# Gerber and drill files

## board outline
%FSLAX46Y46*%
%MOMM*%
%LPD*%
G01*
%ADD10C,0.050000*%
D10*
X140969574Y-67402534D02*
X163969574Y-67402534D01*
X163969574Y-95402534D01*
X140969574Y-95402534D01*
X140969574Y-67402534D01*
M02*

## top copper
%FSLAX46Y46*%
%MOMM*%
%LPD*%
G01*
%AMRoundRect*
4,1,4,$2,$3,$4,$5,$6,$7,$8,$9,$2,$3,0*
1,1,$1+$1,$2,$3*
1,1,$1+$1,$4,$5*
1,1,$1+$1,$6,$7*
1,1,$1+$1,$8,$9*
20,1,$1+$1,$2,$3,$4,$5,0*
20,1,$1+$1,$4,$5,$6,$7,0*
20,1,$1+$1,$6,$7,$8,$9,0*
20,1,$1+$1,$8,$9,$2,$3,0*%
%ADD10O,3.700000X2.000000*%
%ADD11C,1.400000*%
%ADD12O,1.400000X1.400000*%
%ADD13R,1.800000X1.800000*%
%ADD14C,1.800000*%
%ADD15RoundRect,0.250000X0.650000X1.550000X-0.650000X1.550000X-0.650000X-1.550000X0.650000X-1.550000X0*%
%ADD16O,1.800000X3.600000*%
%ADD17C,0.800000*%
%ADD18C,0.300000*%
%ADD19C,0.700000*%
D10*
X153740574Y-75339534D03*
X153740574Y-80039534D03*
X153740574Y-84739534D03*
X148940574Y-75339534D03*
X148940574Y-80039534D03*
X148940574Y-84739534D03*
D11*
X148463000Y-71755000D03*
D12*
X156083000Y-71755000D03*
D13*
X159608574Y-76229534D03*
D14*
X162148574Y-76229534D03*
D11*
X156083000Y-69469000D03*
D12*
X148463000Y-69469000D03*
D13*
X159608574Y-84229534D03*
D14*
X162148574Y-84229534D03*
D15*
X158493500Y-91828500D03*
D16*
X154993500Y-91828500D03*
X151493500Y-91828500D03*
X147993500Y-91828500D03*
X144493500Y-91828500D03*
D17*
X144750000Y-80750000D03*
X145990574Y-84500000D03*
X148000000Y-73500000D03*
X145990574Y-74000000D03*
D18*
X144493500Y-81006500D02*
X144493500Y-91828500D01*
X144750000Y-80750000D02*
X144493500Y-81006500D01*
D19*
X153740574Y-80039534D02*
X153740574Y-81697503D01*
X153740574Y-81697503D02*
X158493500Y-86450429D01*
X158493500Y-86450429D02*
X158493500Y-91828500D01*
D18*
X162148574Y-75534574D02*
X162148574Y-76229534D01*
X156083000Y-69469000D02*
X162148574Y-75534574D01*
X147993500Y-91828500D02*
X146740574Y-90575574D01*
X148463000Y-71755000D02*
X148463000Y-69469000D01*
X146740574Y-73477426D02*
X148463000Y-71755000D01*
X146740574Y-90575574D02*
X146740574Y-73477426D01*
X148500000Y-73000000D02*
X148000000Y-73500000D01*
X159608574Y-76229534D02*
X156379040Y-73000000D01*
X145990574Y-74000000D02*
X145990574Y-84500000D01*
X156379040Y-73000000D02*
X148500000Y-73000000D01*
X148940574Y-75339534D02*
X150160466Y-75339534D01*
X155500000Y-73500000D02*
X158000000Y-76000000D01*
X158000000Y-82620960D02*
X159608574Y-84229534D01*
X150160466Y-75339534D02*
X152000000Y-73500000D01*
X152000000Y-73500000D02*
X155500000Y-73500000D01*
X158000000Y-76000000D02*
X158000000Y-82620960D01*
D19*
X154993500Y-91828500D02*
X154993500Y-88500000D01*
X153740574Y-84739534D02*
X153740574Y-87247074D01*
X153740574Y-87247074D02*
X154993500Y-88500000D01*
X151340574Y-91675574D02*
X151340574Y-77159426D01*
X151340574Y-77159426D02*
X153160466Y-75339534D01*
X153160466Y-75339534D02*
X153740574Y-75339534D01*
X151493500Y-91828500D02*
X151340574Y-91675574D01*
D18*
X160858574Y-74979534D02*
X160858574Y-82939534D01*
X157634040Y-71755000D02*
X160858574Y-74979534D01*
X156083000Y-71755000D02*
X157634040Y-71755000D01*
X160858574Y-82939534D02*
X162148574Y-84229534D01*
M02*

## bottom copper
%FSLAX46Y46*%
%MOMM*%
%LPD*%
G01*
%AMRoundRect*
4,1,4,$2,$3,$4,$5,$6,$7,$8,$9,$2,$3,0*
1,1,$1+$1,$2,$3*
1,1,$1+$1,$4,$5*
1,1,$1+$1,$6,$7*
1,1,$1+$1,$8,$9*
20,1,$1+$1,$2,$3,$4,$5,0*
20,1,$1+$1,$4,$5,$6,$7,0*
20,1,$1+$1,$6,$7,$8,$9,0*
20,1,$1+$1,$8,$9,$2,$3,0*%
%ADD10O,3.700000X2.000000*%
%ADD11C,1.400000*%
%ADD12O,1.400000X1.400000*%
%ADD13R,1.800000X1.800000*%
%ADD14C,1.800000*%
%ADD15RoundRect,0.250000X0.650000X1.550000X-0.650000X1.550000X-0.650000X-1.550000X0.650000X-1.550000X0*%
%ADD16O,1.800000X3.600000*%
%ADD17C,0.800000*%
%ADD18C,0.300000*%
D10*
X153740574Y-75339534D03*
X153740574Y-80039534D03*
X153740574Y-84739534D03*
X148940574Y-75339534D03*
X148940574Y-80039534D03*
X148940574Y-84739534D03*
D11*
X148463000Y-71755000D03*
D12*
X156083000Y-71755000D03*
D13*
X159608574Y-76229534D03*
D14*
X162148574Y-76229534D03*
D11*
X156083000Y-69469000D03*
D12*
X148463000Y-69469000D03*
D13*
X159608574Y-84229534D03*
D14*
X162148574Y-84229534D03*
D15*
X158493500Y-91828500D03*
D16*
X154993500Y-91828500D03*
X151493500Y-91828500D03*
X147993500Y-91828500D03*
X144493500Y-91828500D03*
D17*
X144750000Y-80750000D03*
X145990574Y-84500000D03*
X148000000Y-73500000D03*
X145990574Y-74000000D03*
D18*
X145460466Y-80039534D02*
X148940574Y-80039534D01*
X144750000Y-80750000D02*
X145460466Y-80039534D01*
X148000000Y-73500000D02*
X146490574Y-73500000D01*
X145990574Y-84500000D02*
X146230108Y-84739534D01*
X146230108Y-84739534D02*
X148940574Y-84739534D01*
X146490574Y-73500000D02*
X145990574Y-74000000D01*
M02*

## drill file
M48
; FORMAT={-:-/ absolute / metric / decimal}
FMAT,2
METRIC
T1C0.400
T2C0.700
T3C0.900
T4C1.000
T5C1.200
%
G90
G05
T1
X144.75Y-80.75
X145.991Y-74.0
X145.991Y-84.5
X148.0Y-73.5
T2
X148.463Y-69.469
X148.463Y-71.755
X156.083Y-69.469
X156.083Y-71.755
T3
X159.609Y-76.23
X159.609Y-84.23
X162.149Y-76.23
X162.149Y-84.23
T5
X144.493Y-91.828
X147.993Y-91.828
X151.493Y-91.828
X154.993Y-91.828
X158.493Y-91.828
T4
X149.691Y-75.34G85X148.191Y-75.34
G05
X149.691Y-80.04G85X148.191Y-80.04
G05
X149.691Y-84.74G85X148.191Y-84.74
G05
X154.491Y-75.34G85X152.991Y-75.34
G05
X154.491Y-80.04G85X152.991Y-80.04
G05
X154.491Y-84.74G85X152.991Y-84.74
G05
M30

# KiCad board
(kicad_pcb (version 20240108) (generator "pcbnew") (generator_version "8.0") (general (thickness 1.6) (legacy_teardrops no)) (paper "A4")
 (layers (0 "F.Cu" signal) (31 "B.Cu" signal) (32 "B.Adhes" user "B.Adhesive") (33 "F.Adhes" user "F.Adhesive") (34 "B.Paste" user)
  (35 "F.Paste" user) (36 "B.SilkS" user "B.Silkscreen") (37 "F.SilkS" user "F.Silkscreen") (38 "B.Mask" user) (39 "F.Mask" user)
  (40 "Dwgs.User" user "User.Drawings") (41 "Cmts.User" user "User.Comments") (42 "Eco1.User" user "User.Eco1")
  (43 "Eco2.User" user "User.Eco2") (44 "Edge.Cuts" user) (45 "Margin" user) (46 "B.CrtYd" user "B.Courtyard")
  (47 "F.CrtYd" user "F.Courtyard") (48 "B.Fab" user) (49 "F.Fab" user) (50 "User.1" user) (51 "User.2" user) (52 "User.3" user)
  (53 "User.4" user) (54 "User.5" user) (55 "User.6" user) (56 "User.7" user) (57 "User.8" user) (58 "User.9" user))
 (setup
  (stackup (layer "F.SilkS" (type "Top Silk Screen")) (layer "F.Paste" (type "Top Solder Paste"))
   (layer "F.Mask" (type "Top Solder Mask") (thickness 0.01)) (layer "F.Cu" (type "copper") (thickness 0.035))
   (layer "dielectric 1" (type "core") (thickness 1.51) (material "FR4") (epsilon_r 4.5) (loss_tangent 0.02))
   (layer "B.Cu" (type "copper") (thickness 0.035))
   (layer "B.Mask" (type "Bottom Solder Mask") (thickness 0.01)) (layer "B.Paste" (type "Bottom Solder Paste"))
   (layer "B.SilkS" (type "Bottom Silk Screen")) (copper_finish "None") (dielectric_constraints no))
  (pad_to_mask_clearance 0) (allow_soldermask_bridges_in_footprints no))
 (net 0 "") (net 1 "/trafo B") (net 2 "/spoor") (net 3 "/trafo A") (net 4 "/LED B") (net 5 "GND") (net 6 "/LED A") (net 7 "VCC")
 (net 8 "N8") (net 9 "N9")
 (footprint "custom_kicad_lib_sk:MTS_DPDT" (layer "F.Cu") (at 150.740574 84.039534 -90)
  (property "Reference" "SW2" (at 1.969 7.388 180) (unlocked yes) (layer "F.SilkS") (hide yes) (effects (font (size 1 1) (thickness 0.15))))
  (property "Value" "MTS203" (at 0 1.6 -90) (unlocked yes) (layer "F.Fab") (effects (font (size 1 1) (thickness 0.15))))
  (pad "1" thru_hole oval (at -8.7 -3 270) (size 2 3.7) (drill oval 1 2.5) (layers "*.Cu" "*.Mask") (remove_unused_layers no)
   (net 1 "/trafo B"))
  (pad "2" thru_hole oval (at -4 -3 270) (size 2 3.7) (drill oval 1 2.5) (layers "*.Cu" "*.Mask") (remove_unused_layers no) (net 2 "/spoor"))
  (pad "3" thru_hole oval (at 0.7 -3 270) (size 2 3.7) (drill oval 1 2.5) (layers "*.Cu" "*.Mask") (remove_unused_layers no)
   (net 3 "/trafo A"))
  (pad "4" thru_hole oval (at -8.7 1.8 270) (size 2 3.7) (drill oval 1 2.5) (layers "*.Cu" "*.Mask") (remove_unused_layers no)
   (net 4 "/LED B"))
  (pad "5" thru_hole oval (at -4 1.8 270) (size 2 3.7) (drill oval 1 2.5) (layers "*.Cu" "*.Mask") (remove_unused_layers no) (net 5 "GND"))
  (pad "6" thru_hole oval (at 0.7 1.8 270) (size 2 3.7) (drill oval 1 2.5) (layers "*.Cu" "*.Mask") (remove_unused_layers no)
   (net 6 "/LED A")))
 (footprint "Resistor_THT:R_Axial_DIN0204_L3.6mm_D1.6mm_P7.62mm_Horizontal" (layer "F.Cu") (at 148.463 71.755)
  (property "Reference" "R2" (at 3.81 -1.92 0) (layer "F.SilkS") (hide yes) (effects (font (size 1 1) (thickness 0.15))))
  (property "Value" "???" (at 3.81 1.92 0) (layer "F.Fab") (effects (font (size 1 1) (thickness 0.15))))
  (pad "1" thru_hole circle (at 0 0) (size 1.4 1.4) (drill 0.7) (layers "*.Cu" "*.Mask") (remove_unused_layers no) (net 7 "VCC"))
  (pad "2" thru_hole oval (at 7.62 0) (size 1.4 1.4) (drill 0.7) (layers "*.Cu" "*.Mask") (remove_unused_layers no) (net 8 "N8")))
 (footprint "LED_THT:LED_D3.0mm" (layer "F.Cu") (at 159.608574 76.229534)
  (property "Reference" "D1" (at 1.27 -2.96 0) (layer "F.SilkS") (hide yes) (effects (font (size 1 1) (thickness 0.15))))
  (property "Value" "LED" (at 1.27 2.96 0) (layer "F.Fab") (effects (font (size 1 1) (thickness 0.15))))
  (pad "1" thru_hole rect (at 0 0) (size 1.8 1.8) (drill 0.9) (layers "*.Cu" "*.Mask") (remove_unused_layers no) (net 6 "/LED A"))
  (pad "2" thru_hole circle (at 2.54 0) (size 1.8 1.8) (drill 0.9) (layers "*.Cu" "*.Mask") (remove_unused_layers no) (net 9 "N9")))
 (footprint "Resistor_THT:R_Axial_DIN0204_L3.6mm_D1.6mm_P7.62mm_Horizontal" (layer "F.Cu") (at 156.083 69.469 180)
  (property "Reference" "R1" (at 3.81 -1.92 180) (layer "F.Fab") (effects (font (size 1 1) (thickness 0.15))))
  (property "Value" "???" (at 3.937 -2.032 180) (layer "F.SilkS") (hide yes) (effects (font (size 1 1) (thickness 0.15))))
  (pad "1" thru_hole circle (at 0 0 180) (size 1.4 1.4) (drill 0.7) (layers "*.Cu" "*.Mask") (remove_unused_layers no) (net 9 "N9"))
  (pad "2" thru_hole oval (at 7.62 0 180) (size 1.4 1.4) (drill 0.7) (layers "*.Cu" "*.Mask") (remove_unused_layers no) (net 7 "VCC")))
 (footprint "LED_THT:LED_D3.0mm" (layer "F.Cu") (at 159.608574 84.229534)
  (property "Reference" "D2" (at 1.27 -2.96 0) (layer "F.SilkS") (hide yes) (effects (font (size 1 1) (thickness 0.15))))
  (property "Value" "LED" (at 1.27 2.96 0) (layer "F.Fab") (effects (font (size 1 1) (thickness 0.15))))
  (pad "1" thru_hole rect (at 0 0) (size 1.8 1.8) (drill 0.9) (layers "*.Cu" "*.Mask") (remove_unused_layers no) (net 4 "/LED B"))
  (pad "2" thru_hole circle (at 2.54 0) (size 1.8 1.8) (drill 0.9) (layers "*.Cu" "*.Mask") (remove_unused_layers no) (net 8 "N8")))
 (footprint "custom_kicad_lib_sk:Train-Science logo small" (layer "B.Cu") (at 151.226574 73.025 180)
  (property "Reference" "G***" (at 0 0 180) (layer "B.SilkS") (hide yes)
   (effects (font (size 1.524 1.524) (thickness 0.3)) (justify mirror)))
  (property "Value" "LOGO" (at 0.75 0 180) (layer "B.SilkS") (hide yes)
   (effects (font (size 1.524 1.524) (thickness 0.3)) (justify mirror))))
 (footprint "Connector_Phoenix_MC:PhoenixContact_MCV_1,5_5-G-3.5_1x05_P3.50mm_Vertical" (layer "B.Cu") (at 158.4935 91.8285 180)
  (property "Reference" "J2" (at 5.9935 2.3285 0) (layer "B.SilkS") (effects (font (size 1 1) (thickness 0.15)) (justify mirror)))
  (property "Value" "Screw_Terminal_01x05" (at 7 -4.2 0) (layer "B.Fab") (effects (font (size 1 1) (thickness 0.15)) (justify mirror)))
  (pad "1" thru_hole roundrect (at 0 0 180) (size 1.8 3.6) (drill 1.2) (layers "*.Cu" "*.Mask") (remove_unused_layers no)
   (roundrect_rratio 0.138889) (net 2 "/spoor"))
  (pad "2" thru_hole oval (at 3.5 0 180) (size 1.8 3.6) (drill 1.2) (layers "*.Cu" "*.Mask") (remove_unused_layers no) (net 3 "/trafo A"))
  (pad "3" thru_hole oval (at 7 0 180) (size 1.8 3.6) (drill 1.2) (layers "*.Cu" "*.Mask") (remove_unused_layers no) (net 1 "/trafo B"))
  (pad "4" thru_hole oval (at 10.5 0 180) (size 1.8 3.6) (drill 1.2) (layers "*.Cu" "*.Mask") (remove_unused_layers no) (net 7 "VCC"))
  (pad "5" thru_hole oval (at 14 0 180) (size 1.8 3.6) (drill 1.2) (layers "*.Cu" "*.Mask") (remove_unused_layers no) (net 5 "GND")))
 (gr_rect (start 140.969574 67.402534) (end 163.969574 95.402534) (stroke (width 0.05) (type default)) (fill none) (layer "Edge.Cuts"))
 (segment (start 144.4935 81.0065) (end 144.4935 91.8285) (width 0.3) (layer "F.Cu") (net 5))
 (segment (start 144.75 80.75) (end 144.4935 81.0065) (width 0.3) (layer "F.Cu") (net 5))
 (via (at 144.75 80.75) (size 0.8) (drill 0.4) (layers "F.Cu" "B.Cu") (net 5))
 (segment (start 145.460466 80.039534) (end 148.940574 80.039534) (width 0.3) (layer "B.Cu") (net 5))
 (segment (start 144.75 80.75) (end 145.460466 80.039534) (width 0.3) (layer "B.Cu") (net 5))
 (segment (start 153.740574 80.039534) (end 153.740574 81.697503) (width 0.7) (layer "F.Cu") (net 2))
 (segment (start 153.740574 81.697503) (end 158.4935 86.450429) (width 0.7) (layer "F.Cu") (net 2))
 (segment (start 158.4935 86.450429) (end 158.4935 91.8285) (width 0.7) (layer "F.Cu") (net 2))
 (segment (start 162.148574 75.534574) (end 162.148574 76.229534) (width 0.3) (layer "F.Cu") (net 9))
 (segment (start 156.083 69.469) (end 162.148574 75.534574) (width 0.3) (layer "F.Cu") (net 9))
 (segment (start 147.9935 91.8285) (end 146.740574 90.575574) (width 0.3) (layer "F.Cu") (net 7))
 (segment (start 148.463 71.755) (end 148.463 69.469) (width 0.3) (layer "F.Cu") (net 7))
 (segment (start 146.740574 73.477426) (end 148.463 71.755) (width 0.3) (layer "F.Cu") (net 7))
 (segment (start 146.740574 90.575574) (end 146.740574 73.477426) (width 0.3) (layer "F.Cu") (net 7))
 (segment (start 148.5 73) (end 148 73.5) (width 0.3) (layer "F.Cu") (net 6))
 (segment (start 159.608574 76.229534) (end 156.37904 73) (width 0.3) (layer "F.Cu") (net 6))
 (segment (start 145.990574 74) (end 145.990574 84.5) (width 0.3) (layer "F.Cu") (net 6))
 (segment (start 156.37904 73) (end 148.5 73) (width 0.3) (layer "F.Cu") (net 6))
 (via (at 145.990574 84.5) (size 0.8) (drill 0.4) (layers "F.Cu" "B.Cu") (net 6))
 (via (at 148 73.5) (size 0.8) (drill 0.4) (layers "F.Cu" "B.Cu") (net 6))
 (via (at 145.990574 74) (size 0.8) (drill 0.4) (layers "F.Cu" "B.Cu") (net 6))
 (segment (start 148 73.5) (end 146.490574 73.5) (width 0.3) (layer "B.Cu") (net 6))
 (segment (start 145.990574 84.5) (end 146.230108 84.739534) (width 0.3) (layer "B.Cu") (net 6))
 (segment (start 146.230108 84.739534) (end 148.940574 84.739534) (width 0.3) (layer "B.Cu") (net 6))
 (segment (start 146.490574 73.5) (end 145.990574 74) (width 0.3) (layer "B.Cu") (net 6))
 (segment (start 148.940574 75.339534) (end 150.160466 75.339534) (width 0.3) (layer "F.Cu") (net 4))
 (segment (start 155.5 73.5) (end 158 76) (width 0.3) (layer "F.Cu") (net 4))
 (segment (start 158 82.62096) (end 159.608574 84.229534) (width 0.3) (layer "F.Cu") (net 4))
 (segment (start 150.160466 75.339534) (end 152 73.5) (width 0.3) (layer "F.Cu") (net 4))
 (segment (start 152 73.5) (end 155.5 73.5) (width 0.3) (layer "F.Cu") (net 4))
 (segment (start 158 76) (end 158 82.62096) (width 0.3) (layer "F.Cu") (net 4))
 (segment (start 154.9935 91.8285) (end 154.9935 88.5) (width 0.7) (layer "F.Cu") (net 3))
 (segment (start 153.740574 84.739534) (end 153.740574 87.247074) (width 0.7) (layer "F.Cu") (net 3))
 (segment (start 153.740574 87.247074) (end 154.9935 88.5) (width 0.7) (layer "F.Cu") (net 3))
 (segment (start 151.340574 91.675574) (end 151.340574 77.159426) (width 0.7) (layer "F.Cu") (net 1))
 (segment (start 151.340574 77.159426) (end 153.160466 75.339534) (width 0.7) (layer "F.Cu") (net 1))
 (segment (start 153.160466 75.339534) (end 153.740574 75.339534) (width 0.7) (layer "F.Cu") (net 1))
 (segment (start 151.4935 91.8285) (end 151.340574 91.675574) (width 0.7) (layer "F.Cu") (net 1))
 (segment (start 160.858574 74.979534) (end 160.858574 82.939534) (width 0.3) (layer "F.Cu") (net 8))
 (segment (start 157.63404 71.755) (end 160.858574 74.979534) (width 0.3) (layer "F.Cu") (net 8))
 (segment (start 156.083 71.755) (end 157.63404 71.755) (width 0.3) (layer "F.Cu") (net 8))
 (segment (start 160.858574 82.939534) (end 162.148574 84.229534) (width 0.3) (layer "F.Cu") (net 8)))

